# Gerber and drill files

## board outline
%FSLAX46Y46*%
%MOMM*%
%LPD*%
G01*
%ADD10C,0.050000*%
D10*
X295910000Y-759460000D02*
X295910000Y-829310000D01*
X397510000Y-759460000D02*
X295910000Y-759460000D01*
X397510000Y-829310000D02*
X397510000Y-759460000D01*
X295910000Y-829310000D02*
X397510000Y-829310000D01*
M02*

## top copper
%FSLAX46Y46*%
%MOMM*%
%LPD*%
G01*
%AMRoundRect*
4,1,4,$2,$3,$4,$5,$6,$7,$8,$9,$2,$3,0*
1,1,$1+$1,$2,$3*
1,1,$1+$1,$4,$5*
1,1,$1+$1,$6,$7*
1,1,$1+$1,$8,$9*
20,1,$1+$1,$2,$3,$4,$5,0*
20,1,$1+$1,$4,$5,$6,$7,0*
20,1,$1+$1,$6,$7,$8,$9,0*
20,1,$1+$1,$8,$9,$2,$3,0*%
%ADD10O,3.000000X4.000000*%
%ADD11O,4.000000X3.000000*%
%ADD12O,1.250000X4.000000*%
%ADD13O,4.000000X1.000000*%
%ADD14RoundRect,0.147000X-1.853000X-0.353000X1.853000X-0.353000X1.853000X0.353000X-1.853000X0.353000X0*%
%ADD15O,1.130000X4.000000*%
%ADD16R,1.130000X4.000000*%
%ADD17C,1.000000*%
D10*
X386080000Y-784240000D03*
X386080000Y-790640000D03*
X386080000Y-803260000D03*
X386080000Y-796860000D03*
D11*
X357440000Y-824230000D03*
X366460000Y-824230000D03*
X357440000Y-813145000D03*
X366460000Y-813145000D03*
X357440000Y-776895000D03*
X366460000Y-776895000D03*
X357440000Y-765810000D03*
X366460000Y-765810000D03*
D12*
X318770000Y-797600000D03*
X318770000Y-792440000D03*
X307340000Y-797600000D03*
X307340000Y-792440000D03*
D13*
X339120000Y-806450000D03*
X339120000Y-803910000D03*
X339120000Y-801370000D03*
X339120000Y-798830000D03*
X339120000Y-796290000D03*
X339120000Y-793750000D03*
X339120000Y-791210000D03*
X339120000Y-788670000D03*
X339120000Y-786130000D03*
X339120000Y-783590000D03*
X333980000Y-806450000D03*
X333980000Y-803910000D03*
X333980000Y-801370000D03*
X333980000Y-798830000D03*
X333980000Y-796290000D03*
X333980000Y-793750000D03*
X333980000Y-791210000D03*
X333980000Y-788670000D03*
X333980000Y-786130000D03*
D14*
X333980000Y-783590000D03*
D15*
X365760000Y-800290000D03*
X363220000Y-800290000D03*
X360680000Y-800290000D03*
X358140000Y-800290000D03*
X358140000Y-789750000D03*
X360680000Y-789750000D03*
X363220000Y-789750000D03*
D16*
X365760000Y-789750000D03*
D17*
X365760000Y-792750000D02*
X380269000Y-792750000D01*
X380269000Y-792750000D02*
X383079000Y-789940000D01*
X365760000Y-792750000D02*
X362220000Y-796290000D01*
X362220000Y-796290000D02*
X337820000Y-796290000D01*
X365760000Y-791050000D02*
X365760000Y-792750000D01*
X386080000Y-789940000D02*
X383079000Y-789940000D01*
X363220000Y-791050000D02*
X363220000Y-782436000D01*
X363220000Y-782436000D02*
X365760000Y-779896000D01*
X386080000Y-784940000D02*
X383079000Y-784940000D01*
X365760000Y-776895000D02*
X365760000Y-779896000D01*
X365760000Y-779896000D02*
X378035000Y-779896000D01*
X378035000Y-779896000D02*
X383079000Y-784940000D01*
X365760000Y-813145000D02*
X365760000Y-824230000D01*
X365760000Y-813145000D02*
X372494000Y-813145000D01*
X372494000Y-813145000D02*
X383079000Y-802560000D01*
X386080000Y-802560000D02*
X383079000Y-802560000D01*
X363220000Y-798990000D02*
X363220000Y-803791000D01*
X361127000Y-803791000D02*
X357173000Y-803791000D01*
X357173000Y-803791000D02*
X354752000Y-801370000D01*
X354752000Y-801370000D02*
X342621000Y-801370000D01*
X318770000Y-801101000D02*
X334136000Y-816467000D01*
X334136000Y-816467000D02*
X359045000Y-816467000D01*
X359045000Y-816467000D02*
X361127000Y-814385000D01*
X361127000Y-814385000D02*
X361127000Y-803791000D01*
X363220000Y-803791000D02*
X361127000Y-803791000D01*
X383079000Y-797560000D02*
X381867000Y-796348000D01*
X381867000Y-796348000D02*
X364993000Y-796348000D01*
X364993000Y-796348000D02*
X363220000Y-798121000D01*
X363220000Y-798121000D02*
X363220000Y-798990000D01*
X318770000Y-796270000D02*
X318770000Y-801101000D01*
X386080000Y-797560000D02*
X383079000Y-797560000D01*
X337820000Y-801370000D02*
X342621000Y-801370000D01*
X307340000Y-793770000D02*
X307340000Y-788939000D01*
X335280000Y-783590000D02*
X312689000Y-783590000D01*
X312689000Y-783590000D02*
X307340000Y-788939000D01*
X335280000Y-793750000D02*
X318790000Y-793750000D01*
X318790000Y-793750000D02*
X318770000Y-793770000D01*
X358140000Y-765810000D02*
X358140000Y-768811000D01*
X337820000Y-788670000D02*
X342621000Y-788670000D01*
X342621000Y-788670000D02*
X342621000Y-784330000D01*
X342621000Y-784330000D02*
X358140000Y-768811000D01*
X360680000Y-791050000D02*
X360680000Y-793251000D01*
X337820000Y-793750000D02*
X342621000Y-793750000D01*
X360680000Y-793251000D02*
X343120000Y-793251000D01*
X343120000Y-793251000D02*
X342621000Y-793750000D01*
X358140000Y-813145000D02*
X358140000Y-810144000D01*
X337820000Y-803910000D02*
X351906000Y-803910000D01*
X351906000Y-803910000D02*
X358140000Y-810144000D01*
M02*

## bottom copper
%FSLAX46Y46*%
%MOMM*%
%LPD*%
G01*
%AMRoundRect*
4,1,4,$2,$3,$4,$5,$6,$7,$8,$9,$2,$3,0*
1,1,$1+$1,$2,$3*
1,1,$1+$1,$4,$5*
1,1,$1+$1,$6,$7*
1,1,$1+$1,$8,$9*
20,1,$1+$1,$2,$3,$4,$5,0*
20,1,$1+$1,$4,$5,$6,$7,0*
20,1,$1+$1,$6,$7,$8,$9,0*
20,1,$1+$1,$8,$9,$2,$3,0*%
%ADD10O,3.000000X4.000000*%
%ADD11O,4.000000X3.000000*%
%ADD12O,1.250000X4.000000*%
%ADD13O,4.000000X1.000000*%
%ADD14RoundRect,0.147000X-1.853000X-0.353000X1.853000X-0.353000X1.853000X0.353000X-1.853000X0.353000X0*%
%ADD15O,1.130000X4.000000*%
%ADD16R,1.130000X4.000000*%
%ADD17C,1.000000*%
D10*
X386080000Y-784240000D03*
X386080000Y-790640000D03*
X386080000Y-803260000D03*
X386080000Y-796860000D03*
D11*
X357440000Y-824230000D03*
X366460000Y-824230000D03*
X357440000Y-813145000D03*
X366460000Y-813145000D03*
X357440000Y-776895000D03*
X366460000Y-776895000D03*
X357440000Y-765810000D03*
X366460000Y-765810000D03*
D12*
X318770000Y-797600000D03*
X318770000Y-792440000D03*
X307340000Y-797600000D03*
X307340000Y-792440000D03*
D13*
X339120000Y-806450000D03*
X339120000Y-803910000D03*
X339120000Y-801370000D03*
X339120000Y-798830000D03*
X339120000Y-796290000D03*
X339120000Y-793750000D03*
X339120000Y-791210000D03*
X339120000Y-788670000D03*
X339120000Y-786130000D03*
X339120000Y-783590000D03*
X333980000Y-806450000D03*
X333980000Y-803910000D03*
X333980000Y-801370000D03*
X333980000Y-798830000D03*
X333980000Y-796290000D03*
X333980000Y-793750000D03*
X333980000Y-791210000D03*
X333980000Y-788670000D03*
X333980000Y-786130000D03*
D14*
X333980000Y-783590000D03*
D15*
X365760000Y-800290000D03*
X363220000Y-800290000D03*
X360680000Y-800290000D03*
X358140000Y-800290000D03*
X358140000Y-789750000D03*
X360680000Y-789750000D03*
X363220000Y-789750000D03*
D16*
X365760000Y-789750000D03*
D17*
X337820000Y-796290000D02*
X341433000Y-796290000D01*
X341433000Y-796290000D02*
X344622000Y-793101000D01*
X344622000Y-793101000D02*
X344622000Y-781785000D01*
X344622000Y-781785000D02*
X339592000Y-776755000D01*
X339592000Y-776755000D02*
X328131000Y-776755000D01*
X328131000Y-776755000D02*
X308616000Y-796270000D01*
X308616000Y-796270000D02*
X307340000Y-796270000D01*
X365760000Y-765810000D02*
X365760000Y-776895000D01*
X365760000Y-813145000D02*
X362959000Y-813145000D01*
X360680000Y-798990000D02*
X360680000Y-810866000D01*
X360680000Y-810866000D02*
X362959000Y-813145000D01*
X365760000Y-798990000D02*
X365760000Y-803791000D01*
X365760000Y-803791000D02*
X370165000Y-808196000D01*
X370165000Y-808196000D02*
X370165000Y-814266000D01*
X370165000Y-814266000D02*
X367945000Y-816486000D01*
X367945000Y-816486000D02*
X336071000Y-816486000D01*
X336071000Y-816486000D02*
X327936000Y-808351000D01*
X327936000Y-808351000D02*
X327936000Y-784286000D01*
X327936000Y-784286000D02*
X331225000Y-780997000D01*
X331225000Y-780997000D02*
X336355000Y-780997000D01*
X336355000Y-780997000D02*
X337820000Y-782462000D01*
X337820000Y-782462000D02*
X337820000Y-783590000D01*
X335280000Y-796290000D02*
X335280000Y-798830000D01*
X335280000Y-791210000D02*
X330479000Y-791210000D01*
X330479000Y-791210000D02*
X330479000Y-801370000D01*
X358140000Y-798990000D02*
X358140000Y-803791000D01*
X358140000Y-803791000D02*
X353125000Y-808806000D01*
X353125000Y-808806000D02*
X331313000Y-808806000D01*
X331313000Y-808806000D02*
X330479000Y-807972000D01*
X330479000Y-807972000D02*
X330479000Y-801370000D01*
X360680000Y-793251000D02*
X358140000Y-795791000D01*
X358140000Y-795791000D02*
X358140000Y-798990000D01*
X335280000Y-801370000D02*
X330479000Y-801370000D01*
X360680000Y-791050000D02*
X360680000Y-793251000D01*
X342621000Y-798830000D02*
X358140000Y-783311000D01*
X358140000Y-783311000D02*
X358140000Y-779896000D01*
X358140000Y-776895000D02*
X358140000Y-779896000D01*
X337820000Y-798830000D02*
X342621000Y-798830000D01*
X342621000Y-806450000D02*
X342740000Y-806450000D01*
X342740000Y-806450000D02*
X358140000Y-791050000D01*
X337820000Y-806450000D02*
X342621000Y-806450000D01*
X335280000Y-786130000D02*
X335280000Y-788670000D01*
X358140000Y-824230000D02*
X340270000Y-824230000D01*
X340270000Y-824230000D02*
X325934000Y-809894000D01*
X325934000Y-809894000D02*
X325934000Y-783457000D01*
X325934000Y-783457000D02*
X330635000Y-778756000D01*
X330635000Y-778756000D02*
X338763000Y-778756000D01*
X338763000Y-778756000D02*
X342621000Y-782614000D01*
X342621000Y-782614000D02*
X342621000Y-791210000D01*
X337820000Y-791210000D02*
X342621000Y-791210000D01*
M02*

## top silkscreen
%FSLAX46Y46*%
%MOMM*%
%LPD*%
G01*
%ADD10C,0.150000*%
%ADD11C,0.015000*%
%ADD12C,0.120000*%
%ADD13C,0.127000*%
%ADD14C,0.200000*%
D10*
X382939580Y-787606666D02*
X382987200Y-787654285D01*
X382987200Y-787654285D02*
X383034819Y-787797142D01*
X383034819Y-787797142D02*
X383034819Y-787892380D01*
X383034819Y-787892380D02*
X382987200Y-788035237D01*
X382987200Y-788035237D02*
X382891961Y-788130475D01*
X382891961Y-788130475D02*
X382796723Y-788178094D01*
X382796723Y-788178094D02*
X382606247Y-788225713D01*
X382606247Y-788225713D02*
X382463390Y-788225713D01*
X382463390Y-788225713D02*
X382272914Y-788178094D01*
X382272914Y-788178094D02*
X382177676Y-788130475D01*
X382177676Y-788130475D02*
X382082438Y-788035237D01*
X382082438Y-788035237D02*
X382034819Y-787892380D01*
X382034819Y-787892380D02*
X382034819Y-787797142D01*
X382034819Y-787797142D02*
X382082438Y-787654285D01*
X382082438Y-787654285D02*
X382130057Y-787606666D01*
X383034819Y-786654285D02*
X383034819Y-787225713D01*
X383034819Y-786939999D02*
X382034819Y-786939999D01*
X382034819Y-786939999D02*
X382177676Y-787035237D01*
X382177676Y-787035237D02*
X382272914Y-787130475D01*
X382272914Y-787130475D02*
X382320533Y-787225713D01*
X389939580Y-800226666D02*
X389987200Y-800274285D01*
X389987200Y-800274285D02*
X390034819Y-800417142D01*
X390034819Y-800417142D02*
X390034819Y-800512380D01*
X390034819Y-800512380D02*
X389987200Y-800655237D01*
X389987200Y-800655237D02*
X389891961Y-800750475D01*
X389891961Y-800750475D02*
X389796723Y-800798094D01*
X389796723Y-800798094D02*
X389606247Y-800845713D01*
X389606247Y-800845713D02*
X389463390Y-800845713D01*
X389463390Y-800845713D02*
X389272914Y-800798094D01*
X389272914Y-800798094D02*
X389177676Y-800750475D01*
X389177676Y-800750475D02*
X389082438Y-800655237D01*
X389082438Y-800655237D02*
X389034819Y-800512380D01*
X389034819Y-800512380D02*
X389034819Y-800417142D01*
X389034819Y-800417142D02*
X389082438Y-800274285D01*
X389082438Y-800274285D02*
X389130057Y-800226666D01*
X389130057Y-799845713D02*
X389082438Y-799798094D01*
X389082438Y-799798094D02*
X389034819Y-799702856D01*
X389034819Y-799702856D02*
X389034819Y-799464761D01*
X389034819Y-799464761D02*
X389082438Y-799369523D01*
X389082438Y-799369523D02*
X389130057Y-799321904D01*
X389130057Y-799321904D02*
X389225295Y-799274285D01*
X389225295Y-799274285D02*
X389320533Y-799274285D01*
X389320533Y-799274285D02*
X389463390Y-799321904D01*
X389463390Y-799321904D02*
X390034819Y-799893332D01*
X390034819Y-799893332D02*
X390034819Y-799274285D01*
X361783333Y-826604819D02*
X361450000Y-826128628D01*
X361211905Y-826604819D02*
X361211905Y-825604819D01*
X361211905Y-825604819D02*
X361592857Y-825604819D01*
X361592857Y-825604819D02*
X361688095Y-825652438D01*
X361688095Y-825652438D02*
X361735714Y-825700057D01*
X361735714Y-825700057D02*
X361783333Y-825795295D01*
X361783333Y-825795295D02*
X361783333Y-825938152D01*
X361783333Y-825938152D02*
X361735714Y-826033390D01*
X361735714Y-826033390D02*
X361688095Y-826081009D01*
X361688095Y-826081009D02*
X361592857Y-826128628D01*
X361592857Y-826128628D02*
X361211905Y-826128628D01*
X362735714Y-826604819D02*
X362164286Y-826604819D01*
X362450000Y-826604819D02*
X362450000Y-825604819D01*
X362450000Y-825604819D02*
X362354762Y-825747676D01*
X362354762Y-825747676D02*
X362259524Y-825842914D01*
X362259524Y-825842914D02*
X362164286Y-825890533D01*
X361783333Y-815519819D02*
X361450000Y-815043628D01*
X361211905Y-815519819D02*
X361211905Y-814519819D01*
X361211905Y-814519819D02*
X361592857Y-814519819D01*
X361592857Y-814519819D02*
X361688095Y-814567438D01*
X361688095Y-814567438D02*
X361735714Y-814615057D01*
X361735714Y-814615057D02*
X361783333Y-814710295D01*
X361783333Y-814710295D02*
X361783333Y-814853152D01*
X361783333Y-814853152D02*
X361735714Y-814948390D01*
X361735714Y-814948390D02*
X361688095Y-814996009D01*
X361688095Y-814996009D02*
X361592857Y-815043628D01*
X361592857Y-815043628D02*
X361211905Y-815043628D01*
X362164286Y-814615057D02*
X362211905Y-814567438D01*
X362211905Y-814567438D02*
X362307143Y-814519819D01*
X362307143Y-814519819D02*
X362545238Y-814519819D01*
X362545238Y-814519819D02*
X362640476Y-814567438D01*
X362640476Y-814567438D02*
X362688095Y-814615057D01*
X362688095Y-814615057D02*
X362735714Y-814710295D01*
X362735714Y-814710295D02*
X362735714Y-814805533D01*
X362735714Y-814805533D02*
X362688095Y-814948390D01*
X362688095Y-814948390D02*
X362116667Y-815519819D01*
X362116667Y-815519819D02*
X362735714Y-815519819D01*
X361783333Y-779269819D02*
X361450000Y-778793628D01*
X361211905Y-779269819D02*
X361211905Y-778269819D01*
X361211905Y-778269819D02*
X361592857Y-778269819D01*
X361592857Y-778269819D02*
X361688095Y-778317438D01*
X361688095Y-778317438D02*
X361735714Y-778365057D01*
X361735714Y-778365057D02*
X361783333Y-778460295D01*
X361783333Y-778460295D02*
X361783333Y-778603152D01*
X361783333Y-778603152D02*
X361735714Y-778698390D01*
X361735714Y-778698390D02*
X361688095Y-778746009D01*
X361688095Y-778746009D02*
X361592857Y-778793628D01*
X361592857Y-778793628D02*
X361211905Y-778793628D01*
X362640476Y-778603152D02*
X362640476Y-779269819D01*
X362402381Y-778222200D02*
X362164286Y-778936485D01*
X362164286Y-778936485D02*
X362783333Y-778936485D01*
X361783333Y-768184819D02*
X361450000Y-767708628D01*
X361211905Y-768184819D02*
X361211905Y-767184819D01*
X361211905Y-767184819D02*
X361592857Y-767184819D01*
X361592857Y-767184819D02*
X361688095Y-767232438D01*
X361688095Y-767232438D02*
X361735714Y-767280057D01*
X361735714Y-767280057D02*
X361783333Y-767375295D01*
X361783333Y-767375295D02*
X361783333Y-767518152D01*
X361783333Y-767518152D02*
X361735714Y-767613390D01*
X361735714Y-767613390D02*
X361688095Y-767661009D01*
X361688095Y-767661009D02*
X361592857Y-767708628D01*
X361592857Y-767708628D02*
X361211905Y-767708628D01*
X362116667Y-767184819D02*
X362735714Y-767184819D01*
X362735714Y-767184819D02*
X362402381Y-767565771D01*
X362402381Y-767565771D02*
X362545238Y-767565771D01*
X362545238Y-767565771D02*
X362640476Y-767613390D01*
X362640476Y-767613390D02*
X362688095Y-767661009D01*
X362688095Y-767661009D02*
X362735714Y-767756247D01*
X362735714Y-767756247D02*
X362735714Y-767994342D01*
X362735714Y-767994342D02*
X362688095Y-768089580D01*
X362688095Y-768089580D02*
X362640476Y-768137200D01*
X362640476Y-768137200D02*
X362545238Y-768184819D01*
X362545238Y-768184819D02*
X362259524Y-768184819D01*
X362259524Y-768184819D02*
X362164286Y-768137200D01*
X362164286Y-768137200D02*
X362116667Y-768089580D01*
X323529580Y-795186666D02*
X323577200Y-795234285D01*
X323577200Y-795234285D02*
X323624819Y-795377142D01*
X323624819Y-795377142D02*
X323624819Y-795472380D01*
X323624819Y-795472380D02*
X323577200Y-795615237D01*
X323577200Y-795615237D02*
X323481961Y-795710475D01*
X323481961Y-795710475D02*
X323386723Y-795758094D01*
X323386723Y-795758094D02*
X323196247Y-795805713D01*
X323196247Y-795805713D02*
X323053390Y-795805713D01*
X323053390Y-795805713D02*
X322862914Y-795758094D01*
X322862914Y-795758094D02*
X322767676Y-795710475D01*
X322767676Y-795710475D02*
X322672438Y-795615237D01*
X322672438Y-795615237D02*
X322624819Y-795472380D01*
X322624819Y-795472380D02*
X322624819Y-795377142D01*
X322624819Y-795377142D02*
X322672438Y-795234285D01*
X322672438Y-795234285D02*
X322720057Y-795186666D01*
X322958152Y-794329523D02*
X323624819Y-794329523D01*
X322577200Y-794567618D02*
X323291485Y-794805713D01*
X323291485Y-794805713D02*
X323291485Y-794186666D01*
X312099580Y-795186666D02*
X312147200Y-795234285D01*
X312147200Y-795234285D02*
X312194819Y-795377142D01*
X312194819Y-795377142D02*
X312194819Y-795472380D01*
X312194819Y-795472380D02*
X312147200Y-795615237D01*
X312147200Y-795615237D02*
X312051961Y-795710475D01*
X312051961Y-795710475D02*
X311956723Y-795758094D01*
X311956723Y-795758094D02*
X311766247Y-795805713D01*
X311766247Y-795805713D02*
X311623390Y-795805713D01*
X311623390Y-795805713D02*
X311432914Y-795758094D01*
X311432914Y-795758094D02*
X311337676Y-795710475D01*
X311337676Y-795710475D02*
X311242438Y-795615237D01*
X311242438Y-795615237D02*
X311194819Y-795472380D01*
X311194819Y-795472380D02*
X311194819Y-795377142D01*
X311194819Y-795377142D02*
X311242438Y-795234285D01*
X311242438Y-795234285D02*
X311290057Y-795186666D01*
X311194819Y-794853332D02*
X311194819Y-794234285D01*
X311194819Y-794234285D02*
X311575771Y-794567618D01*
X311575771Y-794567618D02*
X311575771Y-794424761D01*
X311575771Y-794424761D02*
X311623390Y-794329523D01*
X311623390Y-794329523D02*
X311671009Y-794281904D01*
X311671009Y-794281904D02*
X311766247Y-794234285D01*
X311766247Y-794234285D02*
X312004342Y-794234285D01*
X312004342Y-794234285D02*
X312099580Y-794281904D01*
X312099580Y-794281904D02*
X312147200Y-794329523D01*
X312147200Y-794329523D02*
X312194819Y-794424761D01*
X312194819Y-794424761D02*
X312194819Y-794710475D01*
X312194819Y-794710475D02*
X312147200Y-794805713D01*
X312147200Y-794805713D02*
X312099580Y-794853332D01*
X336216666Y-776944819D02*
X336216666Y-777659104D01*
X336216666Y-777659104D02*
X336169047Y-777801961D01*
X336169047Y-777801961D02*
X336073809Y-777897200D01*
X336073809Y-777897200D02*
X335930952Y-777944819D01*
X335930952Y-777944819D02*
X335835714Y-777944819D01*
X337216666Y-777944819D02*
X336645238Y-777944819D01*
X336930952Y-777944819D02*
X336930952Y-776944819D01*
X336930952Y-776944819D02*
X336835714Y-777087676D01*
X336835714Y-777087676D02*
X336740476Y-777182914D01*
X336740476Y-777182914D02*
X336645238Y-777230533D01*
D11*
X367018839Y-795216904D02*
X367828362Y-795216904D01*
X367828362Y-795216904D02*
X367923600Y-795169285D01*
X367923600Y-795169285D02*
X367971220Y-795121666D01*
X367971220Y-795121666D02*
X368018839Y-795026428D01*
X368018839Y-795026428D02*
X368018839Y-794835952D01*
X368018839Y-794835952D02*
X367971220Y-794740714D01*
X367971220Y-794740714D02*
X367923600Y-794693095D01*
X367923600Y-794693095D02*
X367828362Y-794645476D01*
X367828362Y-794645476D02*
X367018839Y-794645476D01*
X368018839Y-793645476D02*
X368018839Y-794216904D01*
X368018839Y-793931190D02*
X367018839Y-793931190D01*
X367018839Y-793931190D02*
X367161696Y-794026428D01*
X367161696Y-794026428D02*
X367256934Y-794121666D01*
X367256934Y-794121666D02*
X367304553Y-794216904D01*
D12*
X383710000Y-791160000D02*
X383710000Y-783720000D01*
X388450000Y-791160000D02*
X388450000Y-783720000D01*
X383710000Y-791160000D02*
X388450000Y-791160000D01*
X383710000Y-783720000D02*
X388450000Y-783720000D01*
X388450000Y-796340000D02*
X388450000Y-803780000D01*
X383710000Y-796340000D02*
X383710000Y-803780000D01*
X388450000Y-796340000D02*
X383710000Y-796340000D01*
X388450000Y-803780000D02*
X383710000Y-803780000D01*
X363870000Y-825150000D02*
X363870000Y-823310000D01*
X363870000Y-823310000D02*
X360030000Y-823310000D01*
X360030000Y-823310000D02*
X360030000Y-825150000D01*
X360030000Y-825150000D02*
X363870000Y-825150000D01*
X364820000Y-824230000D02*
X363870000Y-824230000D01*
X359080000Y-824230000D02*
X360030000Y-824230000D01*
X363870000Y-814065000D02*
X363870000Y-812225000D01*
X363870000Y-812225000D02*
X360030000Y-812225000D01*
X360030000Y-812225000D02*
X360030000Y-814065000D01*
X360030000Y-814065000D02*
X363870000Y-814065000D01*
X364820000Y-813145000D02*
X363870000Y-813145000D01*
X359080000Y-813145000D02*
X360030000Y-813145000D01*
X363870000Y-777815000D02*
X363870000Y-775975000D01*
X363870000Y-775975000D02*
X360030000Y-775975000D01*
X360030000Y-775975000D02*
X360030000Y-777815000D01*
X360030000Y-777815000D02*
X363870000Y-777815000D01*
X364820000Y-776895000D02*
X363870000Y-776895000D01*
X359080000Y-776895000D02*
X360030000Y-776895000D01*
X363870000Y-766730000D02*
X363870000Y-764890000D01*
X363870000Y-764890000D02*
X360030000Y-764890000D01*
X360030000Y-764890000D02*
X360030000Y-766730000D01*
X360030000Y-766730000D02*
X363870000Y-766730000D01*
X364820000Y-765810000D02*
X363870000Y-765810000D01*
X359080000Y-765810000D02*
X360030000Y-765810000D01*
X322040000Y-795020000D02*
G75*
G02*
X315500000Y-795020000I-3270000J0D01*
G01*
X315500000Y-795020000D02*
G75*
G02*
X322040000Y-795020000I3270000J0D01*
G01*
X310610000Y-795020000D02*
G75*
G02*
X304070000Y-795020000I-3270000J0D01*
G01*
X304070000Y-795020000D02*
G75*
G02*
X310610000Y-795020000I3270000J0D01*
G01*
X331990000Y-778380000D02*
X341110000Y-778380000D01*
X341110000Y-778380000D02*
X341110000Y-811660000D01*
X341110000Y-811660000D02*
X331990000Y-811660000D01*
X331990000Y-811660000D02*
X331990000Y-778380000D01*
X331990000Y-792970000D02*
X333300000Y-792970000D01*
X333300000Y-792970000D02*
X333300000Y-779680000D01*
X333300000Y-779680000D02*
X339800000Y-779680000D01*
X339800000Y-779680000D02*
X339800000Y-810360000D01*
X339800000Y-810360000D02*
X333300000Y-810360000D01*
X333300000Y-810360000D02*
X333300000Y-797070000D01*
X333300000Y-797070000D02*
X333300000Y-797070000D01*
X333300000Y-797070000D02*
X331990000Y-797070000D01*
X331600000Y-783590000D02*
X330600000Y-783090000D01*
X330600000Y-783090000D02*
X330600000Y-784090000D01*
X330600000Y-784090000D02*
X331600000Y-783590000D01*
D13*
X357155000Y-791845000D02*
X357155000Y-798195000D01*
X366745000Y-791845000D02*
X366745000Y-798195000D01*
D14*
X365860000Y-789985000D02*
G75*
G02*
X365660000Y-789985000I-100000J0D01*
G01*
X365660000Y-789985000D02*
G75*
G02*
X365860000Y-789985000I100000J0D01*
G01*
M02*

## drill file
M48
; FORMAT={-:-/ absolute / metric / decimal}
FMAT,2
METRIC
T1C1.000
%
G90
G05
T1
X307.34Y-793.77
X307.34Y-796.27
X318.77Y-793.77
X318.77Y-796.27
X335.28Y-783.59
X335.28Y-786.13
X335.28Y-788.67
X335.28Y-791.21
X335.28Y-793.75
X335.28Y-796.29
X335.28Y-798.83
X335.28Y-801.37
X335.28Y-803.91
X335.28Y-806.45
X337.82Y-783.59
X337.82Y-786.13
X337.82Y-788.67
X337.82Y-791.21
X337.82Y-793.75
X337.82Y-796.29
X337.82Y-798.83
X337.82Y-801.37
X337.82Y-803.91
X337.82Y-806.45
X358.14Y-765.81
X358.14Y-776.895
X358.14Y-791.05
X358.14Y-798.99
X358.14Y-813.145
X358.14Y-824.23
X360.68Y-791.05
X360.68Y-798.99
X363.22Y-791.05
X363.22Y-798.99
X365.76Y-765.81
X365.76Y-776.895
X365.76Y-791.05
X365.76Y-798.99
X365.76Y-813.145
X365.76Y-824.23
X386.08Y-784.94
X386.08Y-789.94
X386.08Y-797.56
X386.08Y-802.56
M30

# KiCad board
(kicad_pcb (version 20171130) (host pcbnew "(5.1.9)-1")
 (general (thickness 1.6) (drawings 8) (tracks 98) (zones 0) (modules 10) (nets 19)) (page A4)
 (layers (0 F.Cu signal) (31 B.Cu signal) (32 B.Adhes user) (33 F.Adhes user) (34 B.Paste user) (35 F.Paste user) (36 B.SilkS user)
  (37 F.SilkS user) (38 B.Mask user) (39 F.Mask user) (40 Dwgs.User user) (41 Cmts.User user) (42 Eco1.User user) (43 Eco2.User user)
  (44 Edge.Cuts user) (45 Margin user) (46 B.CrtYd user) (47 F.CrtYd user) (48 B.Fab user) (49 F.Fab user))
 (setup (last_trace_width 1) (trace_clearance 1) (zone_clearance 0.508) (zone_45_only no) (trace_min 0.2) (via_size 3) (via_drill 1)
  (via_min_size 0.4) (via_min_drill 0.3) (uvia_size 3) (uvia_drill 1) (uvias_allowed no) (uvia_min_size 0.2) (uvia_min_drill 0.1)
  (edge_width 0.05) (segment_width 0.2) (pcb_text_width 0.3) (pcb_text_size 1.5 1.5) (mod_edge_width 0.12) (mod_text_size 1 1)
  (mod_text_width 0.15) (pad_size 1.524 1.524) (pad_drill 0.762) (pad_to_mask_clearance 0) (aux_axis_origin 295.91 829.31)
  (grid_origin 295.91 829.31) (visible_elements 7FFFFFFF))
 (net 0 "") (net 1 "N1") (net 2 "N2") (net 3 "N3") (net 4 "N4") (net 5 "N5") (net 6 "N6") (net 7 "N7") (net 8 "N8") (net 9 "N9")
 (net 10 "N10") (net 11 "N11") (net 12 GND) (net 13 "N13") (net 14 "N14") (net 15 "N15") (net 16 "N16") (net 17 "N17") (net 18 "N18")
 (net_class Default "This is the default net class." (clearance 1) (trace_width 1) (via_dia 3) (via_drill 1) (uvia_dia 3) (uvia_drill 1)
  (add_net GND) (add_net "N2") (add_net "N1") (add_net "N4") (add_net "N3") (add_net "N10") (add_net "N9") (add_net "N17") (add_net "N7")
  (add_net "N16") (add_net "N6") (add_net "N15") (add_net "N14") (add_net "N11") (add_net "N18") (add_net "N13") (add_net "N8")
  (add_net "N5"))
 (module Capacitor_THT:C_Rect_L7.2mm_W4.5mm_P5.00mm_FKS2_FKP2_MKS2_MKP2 (layer F.Cu) (at 386.08 789.94 90)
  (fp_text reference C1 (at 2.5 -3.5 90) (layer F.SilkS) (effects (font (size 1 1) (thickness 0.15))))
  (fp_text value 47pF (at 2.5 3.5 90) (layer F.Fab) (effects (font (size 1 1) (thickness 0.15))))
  (fp_line (start -1.22 -2.37) (end 6.22 -2.37) (layer F.SilkS) (width 0.12))
  (fp_line (start -1.22 2.37) (end 6.22 2.37) (layer F.SilkS) (width 0.12))
  (fp_line (start -1.22 -2.37) (end -1.22 2.37) (layer F.SilkS) (width 0.12))
  (fp_line (start 6.22 -2.37) (end 6.22 2.37) (layer F.SilkS) (width 0.12))
  (pad 2 thru_hole oval (at 5 0 90) (size 4 3) (drill 1 (offset 0.7 0)) (layers *.Cu *.Mask) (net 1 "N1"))
  (pad 1 thru_hole oval (at 0 0 90) (size 4 3) (drill 1 (offset -0.7 0)) (layers *.Cu *.Mask) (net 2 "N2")))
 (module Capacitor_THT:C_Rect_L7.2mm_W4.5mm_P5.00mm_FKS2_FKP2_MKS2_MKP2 (layer F.Cu) (at 386.08 797.56 270)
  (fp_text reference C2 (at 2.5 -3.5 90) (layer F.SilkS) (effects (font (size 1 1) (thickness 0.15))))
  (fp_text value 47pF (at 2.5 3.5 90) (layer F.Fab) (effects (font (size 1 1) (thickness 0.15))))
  (fp_line (start -1.22 -2.37) (end 6.22 -2.37) (layer F.SilkS) (width 0.12))
  (fp_line (start -1.22 2.37) (end 6.22 2.37) (layer F.SilkS) (width 0.12))
  (fp_line (start -1.22 -2.37) (end -1.22 2.37) (layer F.SilkS) (width 0.12))
  (fp_line (start 6.22 -2.37) (end 6.22 2.37) (layer F.SilkS) (width 0.12))
  (pad 2 thru_hole oval (at 5 0 270) (size 4 3) (drill 1 (offset 0.7 0)) (layers *.Cu *.Mask) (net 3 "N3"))
  (pad 1 thru_hole oval (at 0 0 270) (size 4 3) (drill 1 (offset -0.7 0)) (layers *.Cu *.Mask) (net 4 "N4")))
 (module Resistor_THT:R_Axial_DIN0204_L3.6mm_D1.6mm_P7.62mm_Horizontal (layer F.Cu) (at 365.76 824.23 180)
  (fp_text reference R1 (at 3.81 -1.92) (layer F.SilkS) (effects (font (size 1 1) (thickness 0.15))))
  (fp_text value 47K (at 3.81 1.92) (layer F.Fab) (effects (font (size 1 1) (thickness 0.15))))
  (fp_line (start 1.89 -0.92) (end 1.89 0.92) (layer F.SilkS) (width 0.12))
  (fp_line (start 1.89 0.92) (end 5.73 0.92) (layer F.SilkS) (width 0.12))
  (fp_line (start 5.73 0.92) (end 5.73 -0.92) (layer F.SilkS) (width 0.12))
  (fp_line (start 5.73 -0.92) (end 1.89 -0.92) (layer F.SilkS) (width 0.12))
  (fp_line (start 0.94 0) (end 1.89 0) (layer F.SilkS) (width 0.12))
  (fp_line (start 6.68 0) (end 5.73 0) (layer F.SilkS) (width 0.12))
  (pad 2 thru_hole oval (at 7.62 0 180) (size 4 3) (drill 1 (offset 0.7 0)) (layers *.Cu *.Mask) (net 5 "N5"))
  (pad 1 thru_hole oval (at 0 0 180) (size 4 3) (drill 1 (offset -0.7 0)) (layers *.Cu *.Mask) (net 3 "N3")))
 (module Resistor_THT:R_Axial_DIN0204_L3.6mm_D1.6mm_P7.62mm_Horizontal (layer F.Cu) (at 365.76 813.145 180)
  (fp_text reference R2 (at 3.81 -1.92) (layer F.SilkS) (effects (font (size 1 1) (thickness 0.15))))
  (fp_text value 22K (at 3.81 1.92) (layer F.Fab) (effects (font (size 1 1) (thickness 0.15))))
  (fp_line (start 1.89 -0.92) (end 1.89 0.92) (layer F.SilkS) (width 0.12))
  (fp_line (start 1.89 0.92) (end 5.73 0.92) (layer F.SilkS) (width 0.12))
  (fp_line (start 5.73 0.92) (end 5.73 -0.92) (layer F.SilkS) (width 0.12))
  (fp_line (start 5.73 -0.92) (end 1.89 -0.92) (layer F.SilkS) (width 0.12))
  (fp_line (start 0.94 0) (end 1.89 0) (layer F.SilkS) (width 0.12))
  (fp_line (start 6.68 0) (end 5.73 0) (layer F.SilkS) (width 0.12))
  (pad 2 thru_hole oval (at 7.62 0 180) (size 4 3) (drill 1 (offset 0.7 0)) (layers *.Cu *.Mask) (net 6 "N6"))
  (pad 1 thru_hole oval (at 0 0 180) (size 4 3) (drill 1 (offset -0.7 0)) (layers *.Cu *.Mask) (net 3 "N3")))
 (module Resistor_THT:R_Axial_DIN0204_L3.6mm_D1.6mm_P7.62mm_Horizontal (layer F.Cu) (at 365.76 776.895 180)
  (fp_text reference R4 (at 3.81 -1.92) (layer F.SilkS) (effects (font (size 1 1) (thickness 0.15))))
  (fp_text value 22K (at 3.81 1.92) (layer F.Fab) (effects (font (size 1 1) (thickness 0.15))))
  (fp_line (start 1.89 -0.92) (end 1.89 0.92) (layer F.SilkS) (width 0.12))
  (fp_line (start 1.89 0.92) (end 5.73 0.92) (layer F.SilkS) (width 0.12))
  (fp_line (start 5.73 0.92) (end 5.73 -0.92) (layer F.SilkS) (width 0.12))
  (fp_line (start 5.73 -0.92) (end 1.89 -0.92) (layer F.SilkS) (width 0.12))
  (fp_line (start 0.94 0) (end 1.89 0) (layer F.SilkS) (width 0.12))
  (fp_line (start 6.68 0) (end 5.73 0) (layer F.SilkS) (width 0.12))
  (pad 2 thru_hole oval (at 7.62 0 180) (size 4 3) (drill 1 (offset 0.7 0)) (layers *.Cu *.Mask) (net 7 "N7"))
  (pad 1 thru_hole oval (at 0 0 180) (size 4 3) (drill 1 (offset -0.7 0)) (layers *.Cu *.Mask) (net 1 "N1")))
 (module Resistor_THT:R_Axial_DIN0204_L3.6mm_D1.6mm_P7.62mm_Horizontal (layer F.Cu) (at 365.76 765.81 180)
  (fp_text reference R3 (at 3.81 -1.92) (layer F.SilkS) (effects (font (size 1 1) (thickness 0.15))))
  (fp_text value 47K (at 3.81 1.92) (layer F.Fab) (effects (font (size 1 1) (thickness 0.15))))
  (fp_line (start 1.89 -0.92) (end 1.89 0.92) (layer F.SilkS) (width 0.12))
  (fp_line (start 1.89 0.92) (end 5.73 0.92) (layer F.SilkS) (width 0.12))
  (fp_line (start 5.73 0.92) (end 5.73 -0.92) (layer F.SilkS) (width 0.12))
  (fp_line (start 5.73 -0.92) (end 1.89 -0.92) (layer F.SilkS) (width 0.12))
  (fp_line (start 0.94 0) (end 1.89 0) (layer F.SilkS) (width 0.12))
  (fp_line (start 6.68 0) (end 5.73 0) (layer F.SilkS) (width 0.12))
  (pad 2 thru_hole oval (at 7.62 0 180) (size 4 3) (drill 1 (offset 0.7 0)) (layers *.Cu *.Mask) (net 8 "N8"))
  (pad 1 thru_hole oval (at 0 0 180) (size 4 3) (drill 1 (offset -0.7 0)) (layers *.Cu *.Mask) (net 1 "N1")))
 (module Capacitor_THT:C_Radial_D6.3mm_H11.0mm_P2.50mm (layer F.Cu) (at 318.77 793.77 270)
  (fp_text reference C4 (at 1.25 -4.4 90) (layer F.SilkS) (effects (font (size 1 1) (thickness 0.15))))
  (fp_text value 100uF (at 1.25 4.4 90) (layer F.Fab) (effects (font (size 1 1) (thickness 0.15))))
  (fp_circle (center 1.25 0) (end 4.52 0) (layer F.SilkS) (width 0.12))
  (pad 2 thru_hole oval (at 2.5 0 270) (size 4 1.25) (drill 1 (offset 1.33 0)) (layers *.Cu *.Mask) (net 4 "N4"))
  (pad 1 thru_hole oval (at 0 0 270) (size 4 1.25) (drill 1 (offset -1.33 0)) (layers *.Cu *.Mask) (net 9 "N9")))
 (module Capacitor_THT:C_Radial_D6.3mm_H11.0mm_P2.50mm (layer F.Cu) (at 307.34 793.77 270)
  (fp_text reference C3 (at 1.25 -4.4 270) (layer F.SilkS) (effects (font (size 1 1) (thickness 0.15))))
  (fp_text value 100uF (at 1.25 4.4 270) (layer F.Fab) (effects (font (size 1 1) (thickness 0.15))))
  (fp_circle (center 1.25 0) (end 4.52 0) (layer F.SilkS) (width 0.12))
  (pad 2 thru_hole oval (at 2.5 0 270) (size 4 1.25) (drill 1 (offset 1.33 0)) (layers *.Cu *.Mask) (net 2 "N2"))
  (pad 1 thru_hole oval (at 0 0 270) (size 4 1.25) (drill 1 (offset -1.33 0)) (layers *.Cu *.Mask) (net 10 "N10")))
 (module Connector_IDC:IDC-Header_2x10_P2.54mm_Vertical (layer F.Cu) (at 335.28 783.59)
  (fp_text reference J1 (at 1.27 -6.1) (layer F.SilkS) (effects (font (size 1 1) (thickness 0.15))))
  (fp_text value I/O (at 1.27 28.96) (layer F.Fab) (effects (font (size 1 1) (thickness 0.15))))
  (fp_line (start -3.29 -5.21) (end 5.83 -5.21) (layer F.SilkS) (width 0.12))
  (fp_line (start 5.83 -5.21) (end 5.83 28.07) (layer F.SilkS) (width 0.12))
  (fp_line (start 5.83 28.07) (end -3.29 28.07) (layer F.SilkS) (width 0.12))
  (fp_line (start -3.29 28.07) (end -3.29 -5.21) (layer F.SilkS) (width 0.12))
  (fp_line (start -3.29 9.38) (end -1.98 9.38) (layer F.SilkS) (width 0.12))
  (fp_line (start -1.98 9.38) (end -1.98 -3.91) (layer F.SilkS) (width 0.12))
  (fp_line (start -1.98 -3.91) (end 4.52 -3.91) (layer F.SilkS) (width 0.12))
  (fp_line (start 4.52 -3.91) (end 4.52 26.77) (layer F.SilkS) (width 0.12))
  (fp_line (start 4.52 26.77) (end -1.98 26.77) (layer F.SilkS) (width 0.12))
  (fp_line (start -1.98 26.77) (end -1.98 13.48) (layer F.SilkS) (width 0.12))
  (fp_line (start -1.98 13.48) (end -1.98 13.48) (layer F.SilkS) (width 0.12))
  (fp_line (start -1.98 13.48) (end -3.29 13.48) (layer F.SilkS) (width 0.12))
  (fp_line (start -3.68 0) (end -4.68 -0.5) (layer F.SilkS) (width 0.12))
  (fp_line (start -4.68 -0.5) (end -4.68 0.5) (layer F.SilkS) (width 0.12))
  (fp_line (start -4.68 0.5) (end -3.68 0) (layer F.SilkS) (width 0.12))
  (pad 20 thru_hole oval (at 2.54 22.86) (size 4 1) (drill 1 (offset 1.3 0)) (layers *.Cu *.Mask) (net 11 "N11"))
  (pad 18 thru_hole oval (at 2.54 20.32) (size 4 1) (drill 1 (offset 1.3 0)) (layers *.Cu *.Mask) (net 6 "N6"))
  (pad 16 thru_hole oval (at 2.54 17.78) (size 4 1) (drill 1 (offset 1.3 0)) (layers *.Cu *.Mask) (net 4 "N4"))
  (pad 14 thru_hole oval (at 2.54 15.24) (size 4 1) (drill 1 (offset 1.3 0)) (layers *.Cu *.Mask) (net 7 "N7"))
  (pad 12 thru_hole oval (at 2.54 12.7) (size 4 1) (drill 1 (offset 1.3 0)) (layers *.Cu *.Mask) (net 2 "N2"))
  (pad 10 thru_hole oval (at 2.54 10.16) (size 4 1) (drill 1 (offset 1.3 0)) (layers *.Cu *.Mask) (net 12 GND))
  (pad 8 thru_hole oval (at 2.54 7.62) (size 4 1) (drill 1 (offset 1.3 0)) (layers *.Cu *.Mask) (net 5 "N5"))
  (pad 6 thru_hole oval (at 2.54 5.08) (size 4 1) (drill 1 (offset 1.3 0)) (layers *.Cu *.Mask) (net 8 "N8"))
  (pad 4 thru_hole oval (at 2.54 2.54) (size 4 1) (drill 1 (offset 1.3 0)) (layers *.Cu *.Mask) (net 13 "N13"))
  (pad 2 thru_hole oval (at 2.54 0) (size 4 1) (drill 1 (offset 1.3 0)) (layers *.Cu *.Mask) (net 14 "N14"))
  (pad 19 thru_hole oval (at 0 22.86) (size 4 1) (drill 1 (offset -1.3 0)) (layers *.Cu *.Mask) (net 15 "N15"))
  (pad 17 thru_hole oval (at 0 20.32) (size 4 1) (drill 1 (offset -1.3 0)) (layers *.Cu *.Mask) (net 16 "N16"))
  (pad 15 thru_hole oval (at 0 17.78) (size 4 1) (drill 1 (offset -1.3 0)) (layers *.Cu *.Mask) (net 12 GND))
  (pad 13 thru_hole oval (at 0 15.24) (size 4 1) (drill 1 (offset -1.3 0)) (layers *.Cu *.Mask) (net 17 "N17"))
  (pad 11 thru_hole oval (at 0 12.7) (size 4 1) (drill 1 (offset -1.3 0)) (layers *.Cu *.Mask) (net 17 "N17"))
  (pad 9 thru_hole oval (at 0 10.16) (size 4 1) (drill 1 (offset -1.3 0)) (layers *.Cu *.Mask) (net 9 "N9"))
  (pad 7 thru_hole oval (at 0 7.62) (size 4 1) (drill 1 (offset -1.3 0)) (layers *.Cu *.Mask) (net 12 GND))
  (pad 5 thru_hole oval (at 0 5.08) (size 4 1) (drill 1 (offset -1.3 0)) (layers *.Cu *.Mask) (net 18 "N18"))
  (pad 3 thru_hole oval (at 0 2.54) (size 4 1) (drill 1 (offset -1.3 0)) (layers *.Cu *.Mask) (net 18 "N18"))
  (pad 1 thru_hole roundrect (at 0 0) (size 4 1) (drill 1 (offset -1.3 0)) (layers *.Cu *.Mask) (roundrect_rratio 0.147) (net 10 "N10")))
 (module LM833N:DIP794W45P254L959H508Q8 (layer F.Cu) (at 361.95 795.02 270)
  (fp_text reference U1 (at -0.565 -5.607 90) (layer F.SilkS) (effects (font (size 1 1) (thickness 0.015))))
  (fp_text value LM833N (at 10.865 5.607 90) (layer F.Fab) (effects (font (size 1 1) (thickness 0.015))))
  (fp_line (start -3.175 4.795) (end 3.175 4.795) (layer F.SilkS) (width 0.127))
  (fp_line (start -3.175 -4.795) (end 3.175 -4.795) (layer F.SilkS) (width 0.127))
  (fp_circle (center -5.035 -3.81) (end -4.935 -3.81) (layer F.SilkS) (width 0.2))
  (pad 8 thru_hole oval (at 3.97 -3.81 270) (size 4 1.13) (drill 1 (offset 1.3 0)) (layers *.Cu *.Mask) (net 14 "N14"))
  (pad 7 thru_hole oval (at 3.97 -1.27 270) (size 4 1.13) (drill 1 (offset 1.3 0)) (layers *.Cu *.Mask) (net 4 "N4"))
  (pad 6 thru_hole oval (at 3.97 1.27 270) (size 4 1.13) (drill 1 (offset 1.3 0)) (layers *.Cu *.Mask) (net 3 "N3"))
  (pad 5 thru_hole oval (at 3.97 3.81 270) (size 4 1.13) (drill 1 (offset 1.3 0)) (layers *.Cu *.Mask) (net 12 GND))
  (pad 4 thru_hole oval (at -3.97 3.81 270) (size 4 1.13) (drill 1 (offset -1.3 0)) (layers *.Cu *.Mask) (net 11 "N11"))
  (pad 3 thru_hole oval (at -3.97 1.27 270) (size 4 1.13) (drill 1 (offset -1.3 0)) (layers *.Cu *.Mask) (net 12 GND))
  (pad 2 thru_hole oval (at -3.97 -1.27 270) (size 4 1.13) (drill 1 (offset -1.3 0)) (layers *.Cu *.Mask) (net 1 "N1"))
  (pad 1 thru_hole rect (at -3.97 -3.81 270) (size 4 1.13) (drill 1 (offset -1.3 0)) (layers *.Cu *.Mask) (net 2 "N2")))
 (gr_line (start 295.91 759.46) (end 295.91 829.31) (layer Edge.Cuts) (width 0.05))
 (gr_line (start 397.51 759.46) (end 295.91 759.46) (layer Edge.Cuts) (width 0.05))
 (gr_line (start 397.51 829.31) (end 397.51 759.46) (layer Edge.Cuts) (width 0.05))
 (gr_line (start 295.91 829.31) (end 397.51 829.31) (layer Edge.Cuts) (width 0.05))
 (segment (start 365.76 792.75) (end 380.269 792.75) (width 1) (layer F.Cu) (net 2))
 (segment (start 380.269 792.75) (end 383.079 789.94) (width 1) (layer F.Cu) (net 2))
 (segment (start 365.76 792.75) (end 362.22 796.29) (width 1) (layer F.Cu) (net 2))
 (segment (start 362.22 796.29) (end 337.82 796.29) (width 1) (layer F.Cu) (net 2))
 (segment (start 365.76 791.05) (end 365.76 792.75) (width 1) (layer F.Cu) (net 2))
 (segment (start 337.82 796.29) (end 341.433 796.29) (width 1) (layer B.Cu) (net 2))
 (segment (start 341.433 796.29) (end 344.622 793.101) (width 1) (layer B.Cu) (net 2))
 (segment (start 344.622 793.101) (end 344.622 781.785) (width 1) (layer B.Cu) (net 2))
 (segment (start 344.622 781.785) (end 339.592 776.755) (width 1) (layer B.Cu) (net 2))
 (segment (start 339.592 776.755) (end 328.131 776.755) (width 1) (layer B.Cu) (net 2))
 (segment (start 328.131 776.755) (end 308.616 796.27) (width 1) (layer B.Cu) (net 2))
 (segment (start 308.616 796.27) (end 307.34 796.27) (width 1) (layer B.Cu) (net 2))
 (segment (start 386.08 789.94) (end 383.079 789.94) (width 1) (layer F.Cu) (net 2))
 (segment (start 363.22 791.05) (end 363.22 782.436) (width 1) (layer F.Cu) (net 1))
 (segment (start 363.22 782.436) (end 365.76 779.896) (width 1) (layer F.Cu) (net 1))
 (segment (start 386.08 784.94) (end 383.079 784.94) (width 1) (layer F.Cu) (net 1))
 (segment (start 365.76 776.895) (end 365.76 779.896) (width 1) (layer F.Cu) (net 1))
 (segment (start 365.76 779.896) (end 378.035 779.896) (width 1) (layer F.Cu) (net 1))
 (segment (start 378.035 779.896) (end 383.079 784.94) (width 1) (layer F.Cu) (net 1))
 (segment (start 365.76 765.81) (end 365.76 776.895) (width 1) (layer B.Cu) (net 1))
 (segment (start 365.76 813.145) (end 365.76 824.23) (width 1) (layer F.Cu) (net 3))
 (segment (start 365.76 813.145) (end 372.494 813.145) (width 1) (layer F.Cu) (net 3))
 (segment (start 372.494 813.145) (end 383.079 802.56) (width 1) (layer F.Cu) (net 3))
 (segment (start 365.76 813.145) (end 362.959 813.145) (width 1) (layer B.Cu) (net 3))
 (segment (start 360.68 798.99) (end 360.68 810.866) (width 1) (layer B.Cu) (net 3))
 (segment (start 360.68 810.866) (end 362.959 813.145) (width 1) (layer B.Cu) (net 3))
 (segment (start 386.08 802.56) (end 383.079 802.56) (width 1) (layer F.Cu) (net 3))
 (segment (start 363.22 798.99) (end 363.22 803.791) (width 1) (layer F.Cu) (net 4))
 (segment (start 361.127 803.791) (end 357.173 803.791) (width 1) (layer F.Cu) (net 4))
 (segment (start 357.173 803.791) (end 354.752 801.37) (width 1) (layer F.Cu) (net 4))
 (segment (start 354.752 801.37) (end 342.621 801.37) (width 1) (layer F.Cu) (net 4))
 (segment (start 318.77 801.101) (end 334.136 816.467) (width 1) (layer F.Cu) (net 4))
 (segment (start 334.136 816.467) (end 359.045 816.467) (width 1) (layer F.Cu) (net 4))
 (segment (start 359.045 816.467) (end 361.127 814.385) (width 1) (layer F.Cu) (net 4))
 (segment (start 361.127 814.385) (end 361.127 803.791) (width 1) (layer F.Cu) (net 4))
 (segment (start 363.22 803.791) (end 361.127 803.791) (width 1) (layer F.Cu) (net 4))
 (segment (start 383.079 797.56) (end 381.867 796.348) (width 1) (layer F.Cu) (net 4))
 (segment (start 381.867 796.348) (end 364.993 796.348) (width 1) (layer F.Cu) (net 4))
 (segment (start 364.993 796.348) (end 363.22 798.121) (width 1) (layer F.Cu) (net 4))
 (segment (start 363.22 798.121) (end 363.22 798.99) (width 1) (layer F.Cu) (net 4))
 (segment (start 318.77 796.27) (end 318.77 801.101) (width 1) (layer F.Cu) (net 4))
 (segment (start 386.08 797.56) (end 383.079 797.56) (width 1) (layer F.Cu) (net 4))
 (segment (start 337.82 801.37) (end 342.621 801.37) (width 1) (layer F.Cu) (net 4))
 (segment (start 307.34 793.77) (end 307.34 788.939) (width 1) (layer F.Cu) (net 10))
 (segment (start 335.28 783.59) (end 312.689 783.59) (width 1) (layer F.Cu) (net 10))
 (segment (start 312.689 783.59) (end 307.34 788.939) (width 1) (layer F.Cu) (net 10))
 (segment (start 335.28 793.75) (end 318.79 793.75) (width 1) (layer F.Cu) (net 9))
 (segment (start 318.79 793.75) (end 318.77 793.77) (width 1) (layer F.Cu) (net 9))
 (segment (start 365.76 798.99) (end 365.76 803.791) (width 1) (layer B.Cu) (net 14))
 (segment (start 365.76 803.791) (end 370.165 808.196) (width 1) (layer B.Cu) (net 14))
 (segment (start 370.165 808.196) (end 370.165 814.266) (width 1) (layer B.Cu) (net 14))
 (segment (start 370.165 814.266) (end 367.945 816.486) (width 1) (layer B.Cu) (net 14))
 (segment (start 367.945 816.486) (end 336.071 816.486) (width 1) (layer B.Cu) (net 14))
 (segment (start 336.071 816.486) (end 327.936 808.351) (width 1) (layer B.Cu) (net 14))
 (segment (start 327.936 808.351) (end 327.936 784.286) (width 1) (layer B.Cu) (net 14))
 (segment (start 327.936 784.286) (end 331.225 780.997) (width 1) (layer B.Cu) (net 14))
 (segment (start 331.225 780.997) (end 336.355 780.997) (width 1) (layer B.Cu) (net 14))
 (segment (start 336.355 780.997) (end 337.82 782.462) (width 1) (layer B.Cu) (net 14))
 (segment (start 337.82 782.462) (end 337.82 783.59) (width 1) (layer B.Cu) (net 14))
 (segment (start 358.14 765.81) (end 358.14 768.811) (width 1) (layer F.Cu) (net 8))
 (segment (start 337.82 788.67) (end 342.621 788.67) (width 1) (layer F.Cu) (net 8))
 (segment (start 342.621 788.67) (end 342.621 784.33) (width 1) (layer F.Cu) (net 8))
 (segment (start 342.621 784.33) (end 358.14 768.811) (width 1) (layer F.Cu) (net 8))
 (segment (start 335.28 796.29) (end 335.28 798.83) (width 1) (layer B.Cu) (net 17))
 (segment (start 360.68 791.05) (end 360.68 793.251) (width 1) (layer F.Cu) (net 12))
 (segment (start 335.28 791.21) (end 330.479 791.21) (width 1) (layer B.Cu) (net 12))
 (segment (start 330.479 791.21) (end 330.479 801.37) (width 1) (layer B.Cu) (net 12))
 (segment (start 358.14 798.99) (end 358.14 803.791) (width 1) (layer B.Cu) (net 12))
 (segment (start 358.14 803.791) (end 353.125 808.806) (width 1) (layer B.Cu) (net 12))
 (segment (start 353.125 808.806) (end 331.313 808.806) (width 1) (layer B.Cu) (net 12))
 (segment (start 331.313 808.806) (end 330.479 807.972) (width 1) (layer B.Cu) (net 12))
 (segment (start 330.479 807.972) (end 330.479 801.37) (width 1) (layer B.Cu) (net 12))
 (segment (start 360.68 793.251) (end 358.14 795.791) (width 1) (layer B.Cu) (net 12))
 (segment (start 358.14 795.791) (end 358.14 798.99) (width 1) (layer B.Cu) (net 12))
 (segment (start 335.28 801.37) (end 330.479 801.37) (width 1) (layer B.Cu) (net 12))
 (segment (start 337.82 793.75) (end 342.621 793.75) (width 1) (layer F.Cu) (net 12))
 (segment (start 360.68 793.251) (end 343.12 793.251) (width 1) (layer F.Cu) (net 12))
 (segment (start 343.12 793.251) (end 342.621 793.75) (width 1) (layer F.Cu) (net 12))
 (segment (start 360.68 791.05) (end 360.68 793.251) (width 1) (layer B.Cu) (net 12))
 (segment (start 342.621 798.83) (end 358.14 783.311) (width 1) (layer B.Cu) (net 7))
 (segment (start 358.14 783.311) (end 358.14 779.896) (width 1) (layer B.Cu) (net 7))
 (segment (start 358.14 776.895) (end 358.14 779.896) (width 1) (layer B.Cu) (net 7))
 (segment (start 337.82 798.83) (end 342.621 798.83) (width 1) (layer B.Cu) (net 7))
 (segment (start 358.14 813.145) (end 358.14 810.144) (width 1) (layer F.Cu) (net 6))
 (segment (start 337.82 803.91) (end 351.906 803.91) (width 1) (layer F.Cu) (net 6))
 (segment (start 351.906 803.91) (end 358.14 810.144) (width 1) (layer F.Cu) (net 6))
 (segment (start 342.621 806.45) (end 342.74 806.45) (width 1) (layer B.Cu) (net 11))
 (segment (start 342.74 806.45) (end 358.14 791.05) (width 1) (layer B.Cu) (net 11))
 (segment (start 337.82 806.45) (end 342.621 806.45) (width 1) (layer B.Cu) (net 11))
 (segment (start 335.28 786.13) (end 335.28 788.67) (width 1) (layer B.Cu) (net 18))
 (segment (start 358.14 824.23) (end 340.27 824.23) (width 1) (layer B.Cu) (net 5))
 (segment (start 340.27 824.23) (end 325.934 809.894) (width 1) (layer B.Cu) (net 5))
 (segment (start 325.934 809.894) (end 325.934 783.457) (width 1) (layer B.Cu) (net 5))
 (segment (start 325.934 783.457) (end 330.635 778.756) (width 1) (layer B.Cu) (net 5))
 (segment (start 330.635 778.756) (end 338.763 778.756) (width 1) (layer B.Cu) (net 5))
 (segment (start 338.763 778.756) (end 342.621 782.614) (width 1) (layer B.Cu) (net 5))
 (segment (start 342.621 782.614) (end 342.621 791.21) (width 1) (layer B.Cu) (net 5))
 (segment (start 337.82 791.21) (end 342.621 791.21) (width 1) (layer B.Cu) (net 5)))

